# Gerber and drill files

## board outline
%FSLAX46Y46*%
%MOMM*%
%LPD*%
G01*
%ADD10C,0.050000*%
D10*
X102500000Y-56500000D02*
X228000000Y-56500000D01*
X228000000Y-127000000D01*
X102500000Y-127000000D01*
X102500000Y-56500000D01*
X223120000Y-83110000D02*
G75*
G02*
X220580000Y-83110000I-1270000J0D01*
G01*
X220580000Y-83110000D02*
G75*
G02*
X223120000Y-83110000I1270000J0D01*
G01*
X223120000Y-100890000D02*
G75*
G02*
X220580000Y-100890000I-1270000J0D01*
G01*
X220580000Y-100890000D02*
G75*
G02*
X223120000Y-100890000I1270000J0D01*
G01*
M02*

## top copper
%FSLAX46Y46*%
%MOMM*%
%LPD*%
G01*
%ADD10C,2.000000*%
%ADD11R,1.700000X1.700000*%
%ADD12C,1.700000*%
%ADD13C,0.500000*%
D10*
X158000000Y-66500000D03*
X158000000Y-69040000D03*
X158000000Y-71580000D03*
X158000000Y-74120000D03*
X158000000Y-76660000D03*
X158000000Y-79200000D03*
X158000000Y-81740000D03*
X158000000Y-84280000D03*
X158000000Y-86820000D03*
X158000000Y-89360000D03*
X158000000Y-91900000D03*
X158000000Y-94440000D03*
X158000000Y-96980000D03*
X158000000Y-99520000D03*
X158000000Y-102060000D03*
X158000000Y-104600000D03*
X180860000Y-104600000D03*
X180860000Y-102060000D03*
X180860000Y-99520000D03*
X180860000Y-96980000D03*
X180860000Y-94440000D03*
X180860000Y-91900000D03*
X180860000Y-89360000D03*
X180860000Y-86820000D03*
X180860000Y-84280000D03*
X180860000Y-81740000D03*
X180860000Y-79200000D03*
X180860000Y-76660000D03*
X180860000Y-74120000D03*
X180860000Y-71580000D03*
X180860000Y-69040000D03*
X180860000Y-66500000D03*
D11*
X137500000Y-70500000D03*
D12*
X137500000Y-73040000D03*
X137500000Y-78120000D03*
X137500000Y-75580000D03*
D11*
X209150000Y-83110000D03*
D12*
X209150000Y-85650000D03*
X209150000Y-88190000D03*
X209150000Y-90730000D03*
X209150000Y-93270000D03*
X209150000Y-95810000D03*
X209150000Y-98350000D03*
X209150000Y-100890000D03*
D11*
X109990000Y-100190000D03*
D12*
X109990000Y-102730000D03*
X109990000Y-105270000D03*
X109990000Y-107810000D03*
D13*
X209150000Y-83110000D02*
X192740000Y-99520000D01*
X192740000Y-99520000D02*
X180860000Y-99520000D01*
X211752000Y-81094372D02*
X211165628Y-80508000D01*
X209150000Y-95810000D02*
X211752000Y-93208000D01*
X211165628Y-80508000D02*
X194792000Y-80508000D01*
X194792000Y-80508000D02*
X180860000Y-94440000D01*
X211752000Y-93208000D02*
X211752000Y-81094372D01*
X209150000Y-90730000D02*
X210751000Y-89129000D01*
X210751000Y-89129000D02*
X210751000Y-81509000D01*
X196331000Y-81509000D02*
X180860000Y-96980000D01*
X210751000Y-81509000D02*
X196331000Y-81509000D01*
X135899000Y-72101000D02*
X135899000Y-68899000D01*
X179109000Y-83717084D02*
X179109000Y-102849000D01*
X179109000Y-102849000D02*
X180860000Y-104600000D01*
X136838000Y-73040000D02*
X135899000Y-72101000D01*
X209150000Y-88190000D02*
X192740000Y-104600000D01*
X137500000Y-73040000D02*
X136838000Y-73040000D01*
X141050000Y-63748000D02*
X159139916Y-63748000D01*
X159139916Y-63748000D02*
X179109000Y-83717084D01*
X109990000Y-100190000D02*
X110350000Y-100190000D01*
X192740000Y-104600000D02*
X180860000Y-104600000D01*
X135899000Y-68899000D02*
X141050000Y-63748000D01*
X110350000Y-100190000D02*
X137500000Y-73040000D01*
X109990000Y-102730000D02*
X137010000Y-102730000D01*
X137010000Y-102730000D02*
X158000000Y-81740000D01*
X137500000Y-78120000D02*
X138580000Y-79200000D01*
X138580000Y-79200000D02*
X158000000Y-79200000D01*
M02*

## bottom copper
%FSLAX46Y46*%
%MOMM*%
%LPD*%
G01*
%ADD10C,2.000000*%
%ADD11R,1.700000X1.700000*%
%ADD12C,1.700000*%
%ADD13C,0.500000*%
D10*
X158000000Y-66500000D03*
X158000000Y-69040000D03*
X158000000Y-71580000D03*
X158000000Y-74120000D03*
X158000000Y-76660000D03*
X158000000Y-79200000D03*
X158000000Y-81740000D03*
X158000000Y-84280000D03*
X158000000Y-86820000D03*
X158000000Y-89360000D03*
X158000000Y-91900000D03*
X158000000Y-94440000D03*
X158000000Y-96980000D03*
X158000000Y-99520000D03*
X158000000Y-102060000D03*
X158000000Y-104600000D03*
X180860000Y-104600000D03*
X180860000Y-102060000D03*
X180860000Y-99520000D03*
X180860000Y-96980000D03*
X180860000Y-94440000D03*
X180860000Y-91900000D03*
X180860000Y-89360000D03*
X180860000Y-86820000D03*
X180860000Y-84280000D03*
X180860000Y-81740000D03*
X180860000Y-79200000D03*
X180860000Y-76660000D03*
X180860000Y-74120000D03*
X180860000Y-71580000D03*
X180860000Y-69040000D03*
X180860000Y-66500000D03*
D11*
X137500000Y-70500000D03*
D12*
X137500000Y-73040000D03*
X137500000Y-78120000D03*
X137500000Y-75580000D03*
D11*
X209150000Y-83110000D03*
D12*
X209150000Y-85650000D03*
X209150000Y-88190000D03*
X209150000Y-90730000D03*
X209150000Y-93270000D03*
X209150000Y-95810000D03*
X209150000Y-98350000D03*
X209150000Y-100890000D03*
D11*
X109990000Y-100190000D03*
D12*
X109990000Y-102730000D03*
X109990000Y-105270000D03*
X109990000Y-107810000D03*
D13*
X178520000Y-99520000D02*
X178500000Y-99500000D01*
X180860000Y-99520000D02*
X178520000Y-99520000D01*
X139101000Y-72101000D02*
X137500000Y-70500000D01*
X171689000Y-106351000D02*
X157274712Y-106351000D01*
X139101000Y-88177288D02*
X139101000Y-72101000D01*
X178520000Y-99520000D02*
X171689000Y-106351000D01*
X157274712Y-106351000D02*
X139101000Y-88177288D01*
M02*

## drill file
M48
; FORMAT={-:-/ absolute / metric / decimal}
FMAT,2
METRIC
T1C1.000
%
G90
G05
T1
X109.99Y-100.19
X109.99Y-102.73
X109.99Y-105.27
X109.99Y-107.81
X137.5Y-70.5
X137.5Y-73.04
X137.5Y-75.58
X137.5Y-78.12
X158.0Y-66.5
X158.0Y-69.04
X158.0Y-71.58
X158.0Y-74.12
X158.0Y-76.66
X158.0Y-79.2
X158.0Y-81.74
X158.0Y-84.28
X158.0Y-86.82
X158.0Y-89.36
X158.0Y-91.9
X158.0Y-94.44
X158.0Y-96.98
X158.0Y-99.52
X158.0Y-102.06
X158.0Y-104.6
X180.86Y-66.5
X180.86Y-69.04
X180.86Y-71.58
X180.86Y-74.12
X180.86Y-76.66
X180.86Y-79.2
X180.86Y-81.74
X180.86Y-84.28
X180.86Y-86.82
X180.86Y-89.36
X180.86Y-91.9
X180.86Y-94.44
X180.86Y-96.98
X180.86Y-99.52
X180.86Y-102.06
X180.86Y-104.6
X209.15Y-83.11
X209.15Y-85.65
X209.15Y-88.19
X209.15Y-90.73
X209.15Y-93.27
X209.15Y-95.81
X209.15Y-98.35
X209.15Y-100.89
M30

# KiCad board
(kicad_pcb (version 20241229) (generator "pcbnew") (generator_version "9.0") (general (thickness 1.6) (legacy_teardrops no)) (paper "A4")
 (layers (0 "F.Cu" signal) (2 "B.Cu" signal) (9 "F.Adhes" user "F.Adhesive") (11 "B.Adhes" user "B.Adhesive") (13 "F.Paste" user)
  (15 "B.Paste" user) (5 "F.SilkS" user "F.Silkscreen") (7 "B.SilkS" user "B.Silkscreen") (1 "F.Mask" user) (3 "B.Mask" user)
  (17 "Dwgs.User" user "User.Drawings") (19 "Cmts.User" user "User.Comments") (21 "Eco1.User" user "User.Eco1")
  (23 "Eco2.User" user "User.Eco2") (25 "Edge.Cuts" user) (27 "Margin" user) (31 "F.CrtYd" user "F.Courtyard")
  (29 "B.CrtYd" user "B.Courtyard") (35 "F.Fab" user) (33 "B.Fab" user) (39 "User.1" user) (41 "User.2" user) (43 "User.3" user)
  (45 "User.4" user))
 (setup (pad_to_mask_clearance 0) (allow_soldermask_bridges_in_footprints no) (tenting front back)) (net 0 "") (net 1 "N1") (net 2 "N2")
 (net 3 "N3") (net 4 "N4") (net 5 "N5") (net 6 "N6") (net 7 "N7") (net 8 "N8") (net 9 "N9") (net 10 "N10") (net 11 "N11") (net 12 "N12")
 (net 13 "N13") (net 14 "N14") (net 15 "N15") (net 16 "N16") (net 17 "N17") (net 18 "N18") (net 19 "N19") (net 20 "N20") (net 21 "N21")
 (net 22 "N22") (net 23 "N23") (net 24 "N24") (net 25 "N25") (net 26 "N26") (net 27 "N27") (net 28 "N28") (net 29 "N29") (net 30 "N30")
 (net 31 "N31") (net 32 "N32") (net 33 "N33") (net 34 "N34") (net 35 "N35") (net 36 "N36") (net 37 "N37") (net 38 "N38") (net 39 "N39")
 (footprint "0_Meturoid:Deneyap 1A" (layer "F.Cu") (at 168.16 91.9)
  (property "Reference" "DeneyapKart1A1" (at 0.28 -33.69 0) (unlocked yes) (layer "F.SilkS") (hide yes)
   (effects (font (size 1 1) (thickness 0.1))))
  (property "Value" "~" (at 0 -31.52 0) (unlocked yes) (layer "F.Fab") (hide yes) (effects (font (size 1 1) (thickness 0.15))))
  (pad "1" thru_hole circle (at -10.16 -25.4) (size 2 2) (drill 1) (layers "*.Cu" "*.Mask") (remove_unused_layers no) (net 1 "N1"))
  (pad "2" thru_hole circle (at -10.16 -22.86) (size 2 2) (drill 1) (layers "*.Cu" "*.Mask") (remove_unused_layers no) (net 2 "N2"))
  (pad "3" thru_hole circle (at -10.16 -20.32) (size 2 2) (drill 1) (layers "*.Cu" "*.Mask") (remove_unused_layers no) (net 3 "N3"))
  (pad "4" thru_hole circle (at -10.16 -17.78) (size 2 2) (drill 1) (layers "*.Cu" "*.Mask") (remove_unused_layers no) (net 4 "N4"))
  (pad "5" thru_hole circle (at -10.16 -15.24) (size 2 2) (drill 1) (layers "*.Cu" "*.Mask") (remove_unused_layers no) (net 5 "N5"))
  (pad "6" thru_hole circle (at -10.16 -12.7) (size 2 2) (drill 1) (layers "*.Cu" "*.Mask") (remove_unused_layers no) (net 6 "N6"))
  (pad "7" thru_hole circle (at -10.16 -10.16) (size 2 2) (drill 1) (layers "*.Cu" "*.Mask") (remove_unused_layers no) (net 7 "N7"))
  (pad "8" thru_hole circle (at -10.16 -7.62) (size 2 2) (drill 1) (layers "*.Cu" "*.Mask") (remove_unused_layers no) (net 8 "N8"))
  (pad "9" thru_hole circle (at -10.16 -5.08) (size 2 2) (drill 1) (layers "*.Cu" "*.Mask") (remove_unused_layers no) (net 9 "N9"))
  (pad "10" thru_hole circle (at -10.16 -2.54) (size 2 2) (drill 1) (layers "*.Cu" "*.Mask") (remove_unused_layers no) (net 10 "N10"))
  (pad "11" thru_hole circle (at -10.16 0) (size 2 2) (drill 1) (layers "*.Cu" "*.Mask") (remove_unused_layers no) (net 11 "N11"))
  (pad "12" thru_hole circle (at -10.16 2.54) (size 2 2) (drill 1) (layers "*.Cu" "*.Mask") (remove_unused_layers no) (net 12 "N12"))
  (pad "13" thru_hole circle (at -10.16 5.08) (size 2 2) (drill 1) (layers "*.Cu" "*.Mask") (remove_unused_layers no) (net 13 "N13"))
  (pad "14" thru_hole circle (at -10.16 7.62) (size 2 2) (drill 1) (layers "*.Cu" "*.Mask") (remove_unused_layers no) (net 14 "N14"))
  (pad "15" thru_hole circle (at -10.16 10.16) (size 2 2) (drill 1) (layers "*.Cu" "*.Mask") (remove_unused_layers no) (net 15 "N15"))
  (pad "16" thru_hole circle (at -10.16 12.7) (size 2 2) (drill 1) (layers "*.Cu" "*.Mask") (remove_unused_layers no) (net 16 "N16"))
  (pad "17" thru_hole circle (at 12.7 12.7) (size 2 2) (drill 1) (layers "*.Cu" "*.Mask") (remove_unused_layers no) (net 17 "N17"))
  (pad "18" thru_hole circle (at 12.7 10.16) (size 2 2) (drill 1) (layers "*.Cu" "*.Mask") (remove_unused_layers no) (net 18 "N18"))
  (pad "19" thru_hole circle (at 12.7 7.62) (size 2 2) (drill 1) (layers "*.Cu" "*.Mask") (remove_unused_layers no) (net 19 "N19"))
  (pad "20" thru_hole circle (at 12.7 5.08) (size 2 2) (drill 1) (layers "*.Cu" "*.Mask") (remove_unused_layers no) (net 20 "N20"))
  (pad "21" thru_hole circle (at 12.7 2.54) (size 2 2) (drill 1) (layers "*.Cu" "*.Mask") (remove_unused_layers no) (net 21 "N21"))
  (pad "22" thru_hole circle (at 12.7 0) (size 2 2) (drill 1) (layers "*.Cu" "*.Mask") (remove_unused_layers no) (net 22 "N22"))
  (pad "23" thru_hole circle (at 12.7 -2.54) (size 2 2) (drill 1) (layers "*.Cu" "*.Mask") (remove_unused_layers no) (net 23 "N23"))
  (pad "24" thru_hole circle (at 12.7 -5.08) (size 2 2) (drill 1) (layers "*.Cu" "*.Mask") (remove_unused_layers no) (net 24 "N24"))
  (pad "25" thru_hole circle (at 12.7 -7.62) (size 2 2) (drill 1) (layers "*.Cu" "*.Mask") (remove_unused_layers no) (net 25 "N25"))
  (pad "26" thru_hole circle (at 12.7 -10.16) (size 2 2) (drill 1) (layers "*.Cu" "*.Mask") (remove_unused_layers no) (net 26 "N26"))
  (pad "27" thru_hole circle (at 12.7 -12.7) (size 2 2) (drill 1) (layers "*.Cu" "*.Mask") (remove_unused_layers no) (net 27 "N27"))
  (pad "28" thru_hole circle (at 12.7 -15.24) (size 2 2) (drill 1) (layers "*.Cu" "*.Mask") (remove_unused_layers no) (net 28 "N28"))
  (pad "29" thru_hole circle (at 12.7 -17.78) (size 2 2) (drill 1) (layers "*.Cu" "*.Mask") (remove_unused_layers no) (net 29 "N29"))
  (pad "30" thru_hole circle (at 12.7 -20.32) (size 2 2) (drill 1) (layers "*.Cu" "*.Mask") (remove_unused_layers no) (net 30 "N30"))
  (pad "31" thru_hole circle (at 12.7 -22.86) (size 2 2) (drill 1) (layers "*.Cu" "*.Mask") (remove_unused_layers no) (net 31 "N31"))
  (pad "32" thru_hole circle (at 12.7 -25.4) (size 2 2) (drill 1) (layers "*.Cu" "*.Mask") (remove_unused_layers no) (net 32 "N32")))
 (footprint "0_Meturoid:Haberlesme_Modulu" (layer "F.Cu") (at 137.5 70.5)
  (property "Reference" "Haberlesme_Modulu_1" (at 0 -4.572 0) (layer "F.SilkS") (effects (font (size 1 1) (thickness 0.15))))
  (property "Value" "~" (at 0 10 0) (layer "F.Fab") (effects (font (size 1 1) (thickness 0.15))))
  (pad "1" thru_hole rect (at 0 0) (size 1.7 1.7) (drill 1) (layers "*.Cu" "*.Mask") (remove_unused_layers no) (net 19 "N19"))
  (pad "2" thru_hole circle (at 0 2.54) (size 1.7 1.7) (drill 1) (layers "*.Cu" "*.Mask") (remove_unused_layers no) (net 17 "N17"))
  (pad "3" thru_hole circle (at 0 7.62) (size 1.7 1.7) (drill 1) (layers "*.Cu" "*.Mask") (remove_unused_layers no) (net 6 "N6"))
  (pad "4" thru_hole circle (at 0 5.08) (size 1.7 1.7) (drill 1) (layers "*.Cu" "*.Mask") (remove_unused_layers no) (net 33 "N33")))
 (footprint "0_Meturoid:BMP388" (layer "F.Cu") (at 209.15 83.11)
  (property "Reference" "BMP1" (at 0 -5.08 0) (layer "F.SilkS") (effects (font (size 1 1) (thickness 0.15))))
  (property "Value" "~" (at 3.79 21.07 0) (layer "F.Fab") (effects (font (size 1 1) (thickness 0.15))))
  (fp_circle (center 12.7 0) (end 12.7 -1.27) (stroke (width 0.05) (type default)) (fill no) (layer "Edge.Cuts"))
  (fp_circle (center 12.7 17.78) (end 13.97 17.78) (stroke (width 0.05) (type default)) (fill no) (layer "Edge.Cuts"))
  (pad "1" thru_hole rect (at 0 0) (size 1.7 1.7) (drill 1) (layers "*.Cu" "*.Mask") (remove_unused_layers no) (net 19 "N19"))
  (pad "2" thru_hole circle (at 0 2.54) (size 1.7 1.7) (drill 1) (layers "*.Cu" "*.Mask") (remove_unused_layers no) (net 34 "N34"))
  (pad "3" thru_hole circle (at 0 5.08) (size 1.7 1.7) (drill 1) (layers "*.Cu" "*.Mask") (remove_unused_layers no) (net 17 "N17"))
  (pad "4" thru_hole circle (at 0 7.62) (size 1.7 1.7) (drill 1) (layers "*.Cu" "*.Mask") (remove_unused_layers no) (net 20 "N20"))
  (pad "5" thru_hole circle (at 0 10.16) (size 1.7 1.7) (drill 1) (layers "*.Cu" "*.Mask") (remove_unused_layers no) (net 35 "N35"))
  (pad "6" thru_hole circle (at 0 12.7) (size 1.7 1.7) (drill 1) (layers "*.Cu" "*.Mask") (remove_unused_layers no) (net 21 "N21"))
  (pad "7" thru_hole circle (at 0 15.24) (size 1.7 1.7) (drill 1) (layers "*.Cu" "*.Mask") (remove_unused_layers no) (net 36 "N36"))
  (pad "8" thru_hole circle (at 0 17.78) (size 1.7 1.7) (drill 1) (layers "*.Cu" "*.Mask") (remove_unused_layers no) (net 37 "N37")))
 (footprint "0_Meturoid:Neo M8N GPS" (layer "F.Cu") (at 109.99 100.19)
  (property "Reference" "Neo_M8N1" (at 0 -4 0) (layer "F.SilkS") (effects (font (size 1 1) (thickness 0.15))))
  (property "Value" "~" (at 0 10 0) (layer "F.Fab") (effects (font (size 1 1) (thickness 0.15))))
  (pad "1" thru_hole rect (at 0 0) (size 1.7 1.7) (drill 1) (layers "*.Cu" "*.Mask") (remove_unused_layers no) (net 17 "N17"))
  (pad "2" thru_hole circle (at 0 2.54) (size 1.7 1.7) (drill 1) (layers "*.Cu" "*.Mask") (remove_unused_layers no) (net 7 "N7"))
  (pad "3" thru_hole circle (at 0 5.08) (size 1.7 1.7) (drill 1) (layers "*.Cu" "*.Mask") (remove_unused_layers no) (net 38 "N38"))
  (pad "4" thru_hole circle (at 0 7.62) (size 1.7 1.7) (drill 1) (layers "*.Cu" "*.Mask") (remove_unused_layers no) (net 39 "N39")))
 (gr_rect (start 102.5 56.5) (end 228 127) (stroke (width 0.05) (type default)) (fill no) (layer "Edge.Cuts"))
 (segment (start 209.15 83.11) (end 192.74 99.52) (width 0.5) (layer "F.Cu") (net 19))
 (segment (start 192.74 99.52) (end 180.86 99.52) (width 0.5) (layer "F.Cu") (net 19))
 (segment (start 178.52 99.52) (end 178.5 99.5) (width 0.5) (layer "B.Cu") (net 19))
 (segment (start 180.86 99.52) (end 178.52 99.52) (width 0.5) (layer "B.Cu") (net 19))
 (segment (start 139.101 72.101) (end 137.5 70.5) (width 0.5) (layer "B.Cu") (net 19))
 (segment (start 171.689 106.351) (end 157.274712 106.351) (width 0.5) (layer "B.Cu") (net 19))
 (segment (start 139.101 88.177288) (end 139.101 72.101) (width 0.5) (layer "B.Cu") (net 19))
 (segment (start 178.52 99.52) (end 171.689 106.351) (width 0.5) (layer "B.Cu") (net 19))
 (segment (start 157.274712 106.351) (end 139.101 88.177288) (width 0.5) (layer "B.Cu") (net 19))
 (segment (start 211.752 81.094372) (end 211.165628 80.508) (width 0.5) (layer "F.Cu") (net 21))
 (segment (start 209.15 95.81) (end 211.752 93.208) (width 0.5) (layer "F.Cu") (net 21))
 (segment (start 211.165628 80.508) (end 194.792 80.508) (width 0.5) (layer "F.Cu") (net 21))
 (segment (start 194.792 80.508) (end 180.86 94.44) (width 0.5) (layer "F.Cu") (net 21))
 (segment (start 211.752 93.208) (end 211.752 81.094372) (width 0.5) (layer "F.Cu") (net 21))
 (segment (start 209.15 90.73) (end 210.751 89.129) (width 0.5) (layer "F.Cu") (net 20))
 (segment (start 210.751 89.129) (end 210.751 81.509) (width 0.5) (layer "F.Cu") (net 20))
 (segment (start 196.331 81.509) (end 180.86 96.98) (width 0.5) (layer "F.Cu") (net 20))
 (segment (start 210.751 81.509) (end 196.331 81.509) (width 0.5) (layer "F.Cu") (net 20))
 (segment (start 135.899 72.101) (end 135.899 68.899) (width 0.5) (layer "F.Cu") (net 17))
 (segment (start 179.109 83.717084) (end 179.109 102.849) (width 0.5) (layer "F.Cu") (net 17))
 (segment (start 179.109 102.849) (end 180.86 104.6) (width 0.5) (layer "F.Cu") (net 17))
 (segment (start 136.838 73.04) (end 135.899 72.101) (width 0.5) (layer "F.Cu") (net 17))
 (segment (start 209.15 88.19) (end 192.74 104.6) (width 0.5) (layer "F.Cu") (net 17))
 (segment (start 137.5 73.04) (end 136.838 73.04) (width 0.5) (layer "F.Cu") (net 17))
 (segment (start 141.05 63.748) (end 159.139916 63.748) (width 0.5) (layer "F.Cu") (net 17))
 (segment (start 159.139916 63.748) (end 179.109 83.717084) (width 0.5) (layer "F.Cu") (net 17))
 (segment (start 109.99 100.19) (end 110.35 100.19) (width 0.5) (layer "F.Cu") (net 17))
 (segment (start 192.74 104.6) (end 180.86 104.6) (width 0.5) (layer "F.Cu") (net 17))
 (segment (start 135.899 68.899) (end 141.05 63.748) (width 0.5) (layer "F.Cu") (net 17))
 (segment (start 110.35 100.19) (end 137.5 73.04) (width 0.5) (layer "F.Cu") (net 17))
 (segment (start 109.99 102.73) (end 137.01 102.73) (width 0.5) (layer "F.Cu") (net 7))
 (segment (start 137.01 102.73) (end 158 81.74) (width 0.5) (layer "F.Cu") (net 7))
 (segment (start 137.5 78.12) (end 138.58 79.2) (width 0.5) (layer "F.Cu") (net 6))
 (segment (start 138.58 79.2) (end 158 79.2) (width 0.5) (layer "F.Cu") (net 6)))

